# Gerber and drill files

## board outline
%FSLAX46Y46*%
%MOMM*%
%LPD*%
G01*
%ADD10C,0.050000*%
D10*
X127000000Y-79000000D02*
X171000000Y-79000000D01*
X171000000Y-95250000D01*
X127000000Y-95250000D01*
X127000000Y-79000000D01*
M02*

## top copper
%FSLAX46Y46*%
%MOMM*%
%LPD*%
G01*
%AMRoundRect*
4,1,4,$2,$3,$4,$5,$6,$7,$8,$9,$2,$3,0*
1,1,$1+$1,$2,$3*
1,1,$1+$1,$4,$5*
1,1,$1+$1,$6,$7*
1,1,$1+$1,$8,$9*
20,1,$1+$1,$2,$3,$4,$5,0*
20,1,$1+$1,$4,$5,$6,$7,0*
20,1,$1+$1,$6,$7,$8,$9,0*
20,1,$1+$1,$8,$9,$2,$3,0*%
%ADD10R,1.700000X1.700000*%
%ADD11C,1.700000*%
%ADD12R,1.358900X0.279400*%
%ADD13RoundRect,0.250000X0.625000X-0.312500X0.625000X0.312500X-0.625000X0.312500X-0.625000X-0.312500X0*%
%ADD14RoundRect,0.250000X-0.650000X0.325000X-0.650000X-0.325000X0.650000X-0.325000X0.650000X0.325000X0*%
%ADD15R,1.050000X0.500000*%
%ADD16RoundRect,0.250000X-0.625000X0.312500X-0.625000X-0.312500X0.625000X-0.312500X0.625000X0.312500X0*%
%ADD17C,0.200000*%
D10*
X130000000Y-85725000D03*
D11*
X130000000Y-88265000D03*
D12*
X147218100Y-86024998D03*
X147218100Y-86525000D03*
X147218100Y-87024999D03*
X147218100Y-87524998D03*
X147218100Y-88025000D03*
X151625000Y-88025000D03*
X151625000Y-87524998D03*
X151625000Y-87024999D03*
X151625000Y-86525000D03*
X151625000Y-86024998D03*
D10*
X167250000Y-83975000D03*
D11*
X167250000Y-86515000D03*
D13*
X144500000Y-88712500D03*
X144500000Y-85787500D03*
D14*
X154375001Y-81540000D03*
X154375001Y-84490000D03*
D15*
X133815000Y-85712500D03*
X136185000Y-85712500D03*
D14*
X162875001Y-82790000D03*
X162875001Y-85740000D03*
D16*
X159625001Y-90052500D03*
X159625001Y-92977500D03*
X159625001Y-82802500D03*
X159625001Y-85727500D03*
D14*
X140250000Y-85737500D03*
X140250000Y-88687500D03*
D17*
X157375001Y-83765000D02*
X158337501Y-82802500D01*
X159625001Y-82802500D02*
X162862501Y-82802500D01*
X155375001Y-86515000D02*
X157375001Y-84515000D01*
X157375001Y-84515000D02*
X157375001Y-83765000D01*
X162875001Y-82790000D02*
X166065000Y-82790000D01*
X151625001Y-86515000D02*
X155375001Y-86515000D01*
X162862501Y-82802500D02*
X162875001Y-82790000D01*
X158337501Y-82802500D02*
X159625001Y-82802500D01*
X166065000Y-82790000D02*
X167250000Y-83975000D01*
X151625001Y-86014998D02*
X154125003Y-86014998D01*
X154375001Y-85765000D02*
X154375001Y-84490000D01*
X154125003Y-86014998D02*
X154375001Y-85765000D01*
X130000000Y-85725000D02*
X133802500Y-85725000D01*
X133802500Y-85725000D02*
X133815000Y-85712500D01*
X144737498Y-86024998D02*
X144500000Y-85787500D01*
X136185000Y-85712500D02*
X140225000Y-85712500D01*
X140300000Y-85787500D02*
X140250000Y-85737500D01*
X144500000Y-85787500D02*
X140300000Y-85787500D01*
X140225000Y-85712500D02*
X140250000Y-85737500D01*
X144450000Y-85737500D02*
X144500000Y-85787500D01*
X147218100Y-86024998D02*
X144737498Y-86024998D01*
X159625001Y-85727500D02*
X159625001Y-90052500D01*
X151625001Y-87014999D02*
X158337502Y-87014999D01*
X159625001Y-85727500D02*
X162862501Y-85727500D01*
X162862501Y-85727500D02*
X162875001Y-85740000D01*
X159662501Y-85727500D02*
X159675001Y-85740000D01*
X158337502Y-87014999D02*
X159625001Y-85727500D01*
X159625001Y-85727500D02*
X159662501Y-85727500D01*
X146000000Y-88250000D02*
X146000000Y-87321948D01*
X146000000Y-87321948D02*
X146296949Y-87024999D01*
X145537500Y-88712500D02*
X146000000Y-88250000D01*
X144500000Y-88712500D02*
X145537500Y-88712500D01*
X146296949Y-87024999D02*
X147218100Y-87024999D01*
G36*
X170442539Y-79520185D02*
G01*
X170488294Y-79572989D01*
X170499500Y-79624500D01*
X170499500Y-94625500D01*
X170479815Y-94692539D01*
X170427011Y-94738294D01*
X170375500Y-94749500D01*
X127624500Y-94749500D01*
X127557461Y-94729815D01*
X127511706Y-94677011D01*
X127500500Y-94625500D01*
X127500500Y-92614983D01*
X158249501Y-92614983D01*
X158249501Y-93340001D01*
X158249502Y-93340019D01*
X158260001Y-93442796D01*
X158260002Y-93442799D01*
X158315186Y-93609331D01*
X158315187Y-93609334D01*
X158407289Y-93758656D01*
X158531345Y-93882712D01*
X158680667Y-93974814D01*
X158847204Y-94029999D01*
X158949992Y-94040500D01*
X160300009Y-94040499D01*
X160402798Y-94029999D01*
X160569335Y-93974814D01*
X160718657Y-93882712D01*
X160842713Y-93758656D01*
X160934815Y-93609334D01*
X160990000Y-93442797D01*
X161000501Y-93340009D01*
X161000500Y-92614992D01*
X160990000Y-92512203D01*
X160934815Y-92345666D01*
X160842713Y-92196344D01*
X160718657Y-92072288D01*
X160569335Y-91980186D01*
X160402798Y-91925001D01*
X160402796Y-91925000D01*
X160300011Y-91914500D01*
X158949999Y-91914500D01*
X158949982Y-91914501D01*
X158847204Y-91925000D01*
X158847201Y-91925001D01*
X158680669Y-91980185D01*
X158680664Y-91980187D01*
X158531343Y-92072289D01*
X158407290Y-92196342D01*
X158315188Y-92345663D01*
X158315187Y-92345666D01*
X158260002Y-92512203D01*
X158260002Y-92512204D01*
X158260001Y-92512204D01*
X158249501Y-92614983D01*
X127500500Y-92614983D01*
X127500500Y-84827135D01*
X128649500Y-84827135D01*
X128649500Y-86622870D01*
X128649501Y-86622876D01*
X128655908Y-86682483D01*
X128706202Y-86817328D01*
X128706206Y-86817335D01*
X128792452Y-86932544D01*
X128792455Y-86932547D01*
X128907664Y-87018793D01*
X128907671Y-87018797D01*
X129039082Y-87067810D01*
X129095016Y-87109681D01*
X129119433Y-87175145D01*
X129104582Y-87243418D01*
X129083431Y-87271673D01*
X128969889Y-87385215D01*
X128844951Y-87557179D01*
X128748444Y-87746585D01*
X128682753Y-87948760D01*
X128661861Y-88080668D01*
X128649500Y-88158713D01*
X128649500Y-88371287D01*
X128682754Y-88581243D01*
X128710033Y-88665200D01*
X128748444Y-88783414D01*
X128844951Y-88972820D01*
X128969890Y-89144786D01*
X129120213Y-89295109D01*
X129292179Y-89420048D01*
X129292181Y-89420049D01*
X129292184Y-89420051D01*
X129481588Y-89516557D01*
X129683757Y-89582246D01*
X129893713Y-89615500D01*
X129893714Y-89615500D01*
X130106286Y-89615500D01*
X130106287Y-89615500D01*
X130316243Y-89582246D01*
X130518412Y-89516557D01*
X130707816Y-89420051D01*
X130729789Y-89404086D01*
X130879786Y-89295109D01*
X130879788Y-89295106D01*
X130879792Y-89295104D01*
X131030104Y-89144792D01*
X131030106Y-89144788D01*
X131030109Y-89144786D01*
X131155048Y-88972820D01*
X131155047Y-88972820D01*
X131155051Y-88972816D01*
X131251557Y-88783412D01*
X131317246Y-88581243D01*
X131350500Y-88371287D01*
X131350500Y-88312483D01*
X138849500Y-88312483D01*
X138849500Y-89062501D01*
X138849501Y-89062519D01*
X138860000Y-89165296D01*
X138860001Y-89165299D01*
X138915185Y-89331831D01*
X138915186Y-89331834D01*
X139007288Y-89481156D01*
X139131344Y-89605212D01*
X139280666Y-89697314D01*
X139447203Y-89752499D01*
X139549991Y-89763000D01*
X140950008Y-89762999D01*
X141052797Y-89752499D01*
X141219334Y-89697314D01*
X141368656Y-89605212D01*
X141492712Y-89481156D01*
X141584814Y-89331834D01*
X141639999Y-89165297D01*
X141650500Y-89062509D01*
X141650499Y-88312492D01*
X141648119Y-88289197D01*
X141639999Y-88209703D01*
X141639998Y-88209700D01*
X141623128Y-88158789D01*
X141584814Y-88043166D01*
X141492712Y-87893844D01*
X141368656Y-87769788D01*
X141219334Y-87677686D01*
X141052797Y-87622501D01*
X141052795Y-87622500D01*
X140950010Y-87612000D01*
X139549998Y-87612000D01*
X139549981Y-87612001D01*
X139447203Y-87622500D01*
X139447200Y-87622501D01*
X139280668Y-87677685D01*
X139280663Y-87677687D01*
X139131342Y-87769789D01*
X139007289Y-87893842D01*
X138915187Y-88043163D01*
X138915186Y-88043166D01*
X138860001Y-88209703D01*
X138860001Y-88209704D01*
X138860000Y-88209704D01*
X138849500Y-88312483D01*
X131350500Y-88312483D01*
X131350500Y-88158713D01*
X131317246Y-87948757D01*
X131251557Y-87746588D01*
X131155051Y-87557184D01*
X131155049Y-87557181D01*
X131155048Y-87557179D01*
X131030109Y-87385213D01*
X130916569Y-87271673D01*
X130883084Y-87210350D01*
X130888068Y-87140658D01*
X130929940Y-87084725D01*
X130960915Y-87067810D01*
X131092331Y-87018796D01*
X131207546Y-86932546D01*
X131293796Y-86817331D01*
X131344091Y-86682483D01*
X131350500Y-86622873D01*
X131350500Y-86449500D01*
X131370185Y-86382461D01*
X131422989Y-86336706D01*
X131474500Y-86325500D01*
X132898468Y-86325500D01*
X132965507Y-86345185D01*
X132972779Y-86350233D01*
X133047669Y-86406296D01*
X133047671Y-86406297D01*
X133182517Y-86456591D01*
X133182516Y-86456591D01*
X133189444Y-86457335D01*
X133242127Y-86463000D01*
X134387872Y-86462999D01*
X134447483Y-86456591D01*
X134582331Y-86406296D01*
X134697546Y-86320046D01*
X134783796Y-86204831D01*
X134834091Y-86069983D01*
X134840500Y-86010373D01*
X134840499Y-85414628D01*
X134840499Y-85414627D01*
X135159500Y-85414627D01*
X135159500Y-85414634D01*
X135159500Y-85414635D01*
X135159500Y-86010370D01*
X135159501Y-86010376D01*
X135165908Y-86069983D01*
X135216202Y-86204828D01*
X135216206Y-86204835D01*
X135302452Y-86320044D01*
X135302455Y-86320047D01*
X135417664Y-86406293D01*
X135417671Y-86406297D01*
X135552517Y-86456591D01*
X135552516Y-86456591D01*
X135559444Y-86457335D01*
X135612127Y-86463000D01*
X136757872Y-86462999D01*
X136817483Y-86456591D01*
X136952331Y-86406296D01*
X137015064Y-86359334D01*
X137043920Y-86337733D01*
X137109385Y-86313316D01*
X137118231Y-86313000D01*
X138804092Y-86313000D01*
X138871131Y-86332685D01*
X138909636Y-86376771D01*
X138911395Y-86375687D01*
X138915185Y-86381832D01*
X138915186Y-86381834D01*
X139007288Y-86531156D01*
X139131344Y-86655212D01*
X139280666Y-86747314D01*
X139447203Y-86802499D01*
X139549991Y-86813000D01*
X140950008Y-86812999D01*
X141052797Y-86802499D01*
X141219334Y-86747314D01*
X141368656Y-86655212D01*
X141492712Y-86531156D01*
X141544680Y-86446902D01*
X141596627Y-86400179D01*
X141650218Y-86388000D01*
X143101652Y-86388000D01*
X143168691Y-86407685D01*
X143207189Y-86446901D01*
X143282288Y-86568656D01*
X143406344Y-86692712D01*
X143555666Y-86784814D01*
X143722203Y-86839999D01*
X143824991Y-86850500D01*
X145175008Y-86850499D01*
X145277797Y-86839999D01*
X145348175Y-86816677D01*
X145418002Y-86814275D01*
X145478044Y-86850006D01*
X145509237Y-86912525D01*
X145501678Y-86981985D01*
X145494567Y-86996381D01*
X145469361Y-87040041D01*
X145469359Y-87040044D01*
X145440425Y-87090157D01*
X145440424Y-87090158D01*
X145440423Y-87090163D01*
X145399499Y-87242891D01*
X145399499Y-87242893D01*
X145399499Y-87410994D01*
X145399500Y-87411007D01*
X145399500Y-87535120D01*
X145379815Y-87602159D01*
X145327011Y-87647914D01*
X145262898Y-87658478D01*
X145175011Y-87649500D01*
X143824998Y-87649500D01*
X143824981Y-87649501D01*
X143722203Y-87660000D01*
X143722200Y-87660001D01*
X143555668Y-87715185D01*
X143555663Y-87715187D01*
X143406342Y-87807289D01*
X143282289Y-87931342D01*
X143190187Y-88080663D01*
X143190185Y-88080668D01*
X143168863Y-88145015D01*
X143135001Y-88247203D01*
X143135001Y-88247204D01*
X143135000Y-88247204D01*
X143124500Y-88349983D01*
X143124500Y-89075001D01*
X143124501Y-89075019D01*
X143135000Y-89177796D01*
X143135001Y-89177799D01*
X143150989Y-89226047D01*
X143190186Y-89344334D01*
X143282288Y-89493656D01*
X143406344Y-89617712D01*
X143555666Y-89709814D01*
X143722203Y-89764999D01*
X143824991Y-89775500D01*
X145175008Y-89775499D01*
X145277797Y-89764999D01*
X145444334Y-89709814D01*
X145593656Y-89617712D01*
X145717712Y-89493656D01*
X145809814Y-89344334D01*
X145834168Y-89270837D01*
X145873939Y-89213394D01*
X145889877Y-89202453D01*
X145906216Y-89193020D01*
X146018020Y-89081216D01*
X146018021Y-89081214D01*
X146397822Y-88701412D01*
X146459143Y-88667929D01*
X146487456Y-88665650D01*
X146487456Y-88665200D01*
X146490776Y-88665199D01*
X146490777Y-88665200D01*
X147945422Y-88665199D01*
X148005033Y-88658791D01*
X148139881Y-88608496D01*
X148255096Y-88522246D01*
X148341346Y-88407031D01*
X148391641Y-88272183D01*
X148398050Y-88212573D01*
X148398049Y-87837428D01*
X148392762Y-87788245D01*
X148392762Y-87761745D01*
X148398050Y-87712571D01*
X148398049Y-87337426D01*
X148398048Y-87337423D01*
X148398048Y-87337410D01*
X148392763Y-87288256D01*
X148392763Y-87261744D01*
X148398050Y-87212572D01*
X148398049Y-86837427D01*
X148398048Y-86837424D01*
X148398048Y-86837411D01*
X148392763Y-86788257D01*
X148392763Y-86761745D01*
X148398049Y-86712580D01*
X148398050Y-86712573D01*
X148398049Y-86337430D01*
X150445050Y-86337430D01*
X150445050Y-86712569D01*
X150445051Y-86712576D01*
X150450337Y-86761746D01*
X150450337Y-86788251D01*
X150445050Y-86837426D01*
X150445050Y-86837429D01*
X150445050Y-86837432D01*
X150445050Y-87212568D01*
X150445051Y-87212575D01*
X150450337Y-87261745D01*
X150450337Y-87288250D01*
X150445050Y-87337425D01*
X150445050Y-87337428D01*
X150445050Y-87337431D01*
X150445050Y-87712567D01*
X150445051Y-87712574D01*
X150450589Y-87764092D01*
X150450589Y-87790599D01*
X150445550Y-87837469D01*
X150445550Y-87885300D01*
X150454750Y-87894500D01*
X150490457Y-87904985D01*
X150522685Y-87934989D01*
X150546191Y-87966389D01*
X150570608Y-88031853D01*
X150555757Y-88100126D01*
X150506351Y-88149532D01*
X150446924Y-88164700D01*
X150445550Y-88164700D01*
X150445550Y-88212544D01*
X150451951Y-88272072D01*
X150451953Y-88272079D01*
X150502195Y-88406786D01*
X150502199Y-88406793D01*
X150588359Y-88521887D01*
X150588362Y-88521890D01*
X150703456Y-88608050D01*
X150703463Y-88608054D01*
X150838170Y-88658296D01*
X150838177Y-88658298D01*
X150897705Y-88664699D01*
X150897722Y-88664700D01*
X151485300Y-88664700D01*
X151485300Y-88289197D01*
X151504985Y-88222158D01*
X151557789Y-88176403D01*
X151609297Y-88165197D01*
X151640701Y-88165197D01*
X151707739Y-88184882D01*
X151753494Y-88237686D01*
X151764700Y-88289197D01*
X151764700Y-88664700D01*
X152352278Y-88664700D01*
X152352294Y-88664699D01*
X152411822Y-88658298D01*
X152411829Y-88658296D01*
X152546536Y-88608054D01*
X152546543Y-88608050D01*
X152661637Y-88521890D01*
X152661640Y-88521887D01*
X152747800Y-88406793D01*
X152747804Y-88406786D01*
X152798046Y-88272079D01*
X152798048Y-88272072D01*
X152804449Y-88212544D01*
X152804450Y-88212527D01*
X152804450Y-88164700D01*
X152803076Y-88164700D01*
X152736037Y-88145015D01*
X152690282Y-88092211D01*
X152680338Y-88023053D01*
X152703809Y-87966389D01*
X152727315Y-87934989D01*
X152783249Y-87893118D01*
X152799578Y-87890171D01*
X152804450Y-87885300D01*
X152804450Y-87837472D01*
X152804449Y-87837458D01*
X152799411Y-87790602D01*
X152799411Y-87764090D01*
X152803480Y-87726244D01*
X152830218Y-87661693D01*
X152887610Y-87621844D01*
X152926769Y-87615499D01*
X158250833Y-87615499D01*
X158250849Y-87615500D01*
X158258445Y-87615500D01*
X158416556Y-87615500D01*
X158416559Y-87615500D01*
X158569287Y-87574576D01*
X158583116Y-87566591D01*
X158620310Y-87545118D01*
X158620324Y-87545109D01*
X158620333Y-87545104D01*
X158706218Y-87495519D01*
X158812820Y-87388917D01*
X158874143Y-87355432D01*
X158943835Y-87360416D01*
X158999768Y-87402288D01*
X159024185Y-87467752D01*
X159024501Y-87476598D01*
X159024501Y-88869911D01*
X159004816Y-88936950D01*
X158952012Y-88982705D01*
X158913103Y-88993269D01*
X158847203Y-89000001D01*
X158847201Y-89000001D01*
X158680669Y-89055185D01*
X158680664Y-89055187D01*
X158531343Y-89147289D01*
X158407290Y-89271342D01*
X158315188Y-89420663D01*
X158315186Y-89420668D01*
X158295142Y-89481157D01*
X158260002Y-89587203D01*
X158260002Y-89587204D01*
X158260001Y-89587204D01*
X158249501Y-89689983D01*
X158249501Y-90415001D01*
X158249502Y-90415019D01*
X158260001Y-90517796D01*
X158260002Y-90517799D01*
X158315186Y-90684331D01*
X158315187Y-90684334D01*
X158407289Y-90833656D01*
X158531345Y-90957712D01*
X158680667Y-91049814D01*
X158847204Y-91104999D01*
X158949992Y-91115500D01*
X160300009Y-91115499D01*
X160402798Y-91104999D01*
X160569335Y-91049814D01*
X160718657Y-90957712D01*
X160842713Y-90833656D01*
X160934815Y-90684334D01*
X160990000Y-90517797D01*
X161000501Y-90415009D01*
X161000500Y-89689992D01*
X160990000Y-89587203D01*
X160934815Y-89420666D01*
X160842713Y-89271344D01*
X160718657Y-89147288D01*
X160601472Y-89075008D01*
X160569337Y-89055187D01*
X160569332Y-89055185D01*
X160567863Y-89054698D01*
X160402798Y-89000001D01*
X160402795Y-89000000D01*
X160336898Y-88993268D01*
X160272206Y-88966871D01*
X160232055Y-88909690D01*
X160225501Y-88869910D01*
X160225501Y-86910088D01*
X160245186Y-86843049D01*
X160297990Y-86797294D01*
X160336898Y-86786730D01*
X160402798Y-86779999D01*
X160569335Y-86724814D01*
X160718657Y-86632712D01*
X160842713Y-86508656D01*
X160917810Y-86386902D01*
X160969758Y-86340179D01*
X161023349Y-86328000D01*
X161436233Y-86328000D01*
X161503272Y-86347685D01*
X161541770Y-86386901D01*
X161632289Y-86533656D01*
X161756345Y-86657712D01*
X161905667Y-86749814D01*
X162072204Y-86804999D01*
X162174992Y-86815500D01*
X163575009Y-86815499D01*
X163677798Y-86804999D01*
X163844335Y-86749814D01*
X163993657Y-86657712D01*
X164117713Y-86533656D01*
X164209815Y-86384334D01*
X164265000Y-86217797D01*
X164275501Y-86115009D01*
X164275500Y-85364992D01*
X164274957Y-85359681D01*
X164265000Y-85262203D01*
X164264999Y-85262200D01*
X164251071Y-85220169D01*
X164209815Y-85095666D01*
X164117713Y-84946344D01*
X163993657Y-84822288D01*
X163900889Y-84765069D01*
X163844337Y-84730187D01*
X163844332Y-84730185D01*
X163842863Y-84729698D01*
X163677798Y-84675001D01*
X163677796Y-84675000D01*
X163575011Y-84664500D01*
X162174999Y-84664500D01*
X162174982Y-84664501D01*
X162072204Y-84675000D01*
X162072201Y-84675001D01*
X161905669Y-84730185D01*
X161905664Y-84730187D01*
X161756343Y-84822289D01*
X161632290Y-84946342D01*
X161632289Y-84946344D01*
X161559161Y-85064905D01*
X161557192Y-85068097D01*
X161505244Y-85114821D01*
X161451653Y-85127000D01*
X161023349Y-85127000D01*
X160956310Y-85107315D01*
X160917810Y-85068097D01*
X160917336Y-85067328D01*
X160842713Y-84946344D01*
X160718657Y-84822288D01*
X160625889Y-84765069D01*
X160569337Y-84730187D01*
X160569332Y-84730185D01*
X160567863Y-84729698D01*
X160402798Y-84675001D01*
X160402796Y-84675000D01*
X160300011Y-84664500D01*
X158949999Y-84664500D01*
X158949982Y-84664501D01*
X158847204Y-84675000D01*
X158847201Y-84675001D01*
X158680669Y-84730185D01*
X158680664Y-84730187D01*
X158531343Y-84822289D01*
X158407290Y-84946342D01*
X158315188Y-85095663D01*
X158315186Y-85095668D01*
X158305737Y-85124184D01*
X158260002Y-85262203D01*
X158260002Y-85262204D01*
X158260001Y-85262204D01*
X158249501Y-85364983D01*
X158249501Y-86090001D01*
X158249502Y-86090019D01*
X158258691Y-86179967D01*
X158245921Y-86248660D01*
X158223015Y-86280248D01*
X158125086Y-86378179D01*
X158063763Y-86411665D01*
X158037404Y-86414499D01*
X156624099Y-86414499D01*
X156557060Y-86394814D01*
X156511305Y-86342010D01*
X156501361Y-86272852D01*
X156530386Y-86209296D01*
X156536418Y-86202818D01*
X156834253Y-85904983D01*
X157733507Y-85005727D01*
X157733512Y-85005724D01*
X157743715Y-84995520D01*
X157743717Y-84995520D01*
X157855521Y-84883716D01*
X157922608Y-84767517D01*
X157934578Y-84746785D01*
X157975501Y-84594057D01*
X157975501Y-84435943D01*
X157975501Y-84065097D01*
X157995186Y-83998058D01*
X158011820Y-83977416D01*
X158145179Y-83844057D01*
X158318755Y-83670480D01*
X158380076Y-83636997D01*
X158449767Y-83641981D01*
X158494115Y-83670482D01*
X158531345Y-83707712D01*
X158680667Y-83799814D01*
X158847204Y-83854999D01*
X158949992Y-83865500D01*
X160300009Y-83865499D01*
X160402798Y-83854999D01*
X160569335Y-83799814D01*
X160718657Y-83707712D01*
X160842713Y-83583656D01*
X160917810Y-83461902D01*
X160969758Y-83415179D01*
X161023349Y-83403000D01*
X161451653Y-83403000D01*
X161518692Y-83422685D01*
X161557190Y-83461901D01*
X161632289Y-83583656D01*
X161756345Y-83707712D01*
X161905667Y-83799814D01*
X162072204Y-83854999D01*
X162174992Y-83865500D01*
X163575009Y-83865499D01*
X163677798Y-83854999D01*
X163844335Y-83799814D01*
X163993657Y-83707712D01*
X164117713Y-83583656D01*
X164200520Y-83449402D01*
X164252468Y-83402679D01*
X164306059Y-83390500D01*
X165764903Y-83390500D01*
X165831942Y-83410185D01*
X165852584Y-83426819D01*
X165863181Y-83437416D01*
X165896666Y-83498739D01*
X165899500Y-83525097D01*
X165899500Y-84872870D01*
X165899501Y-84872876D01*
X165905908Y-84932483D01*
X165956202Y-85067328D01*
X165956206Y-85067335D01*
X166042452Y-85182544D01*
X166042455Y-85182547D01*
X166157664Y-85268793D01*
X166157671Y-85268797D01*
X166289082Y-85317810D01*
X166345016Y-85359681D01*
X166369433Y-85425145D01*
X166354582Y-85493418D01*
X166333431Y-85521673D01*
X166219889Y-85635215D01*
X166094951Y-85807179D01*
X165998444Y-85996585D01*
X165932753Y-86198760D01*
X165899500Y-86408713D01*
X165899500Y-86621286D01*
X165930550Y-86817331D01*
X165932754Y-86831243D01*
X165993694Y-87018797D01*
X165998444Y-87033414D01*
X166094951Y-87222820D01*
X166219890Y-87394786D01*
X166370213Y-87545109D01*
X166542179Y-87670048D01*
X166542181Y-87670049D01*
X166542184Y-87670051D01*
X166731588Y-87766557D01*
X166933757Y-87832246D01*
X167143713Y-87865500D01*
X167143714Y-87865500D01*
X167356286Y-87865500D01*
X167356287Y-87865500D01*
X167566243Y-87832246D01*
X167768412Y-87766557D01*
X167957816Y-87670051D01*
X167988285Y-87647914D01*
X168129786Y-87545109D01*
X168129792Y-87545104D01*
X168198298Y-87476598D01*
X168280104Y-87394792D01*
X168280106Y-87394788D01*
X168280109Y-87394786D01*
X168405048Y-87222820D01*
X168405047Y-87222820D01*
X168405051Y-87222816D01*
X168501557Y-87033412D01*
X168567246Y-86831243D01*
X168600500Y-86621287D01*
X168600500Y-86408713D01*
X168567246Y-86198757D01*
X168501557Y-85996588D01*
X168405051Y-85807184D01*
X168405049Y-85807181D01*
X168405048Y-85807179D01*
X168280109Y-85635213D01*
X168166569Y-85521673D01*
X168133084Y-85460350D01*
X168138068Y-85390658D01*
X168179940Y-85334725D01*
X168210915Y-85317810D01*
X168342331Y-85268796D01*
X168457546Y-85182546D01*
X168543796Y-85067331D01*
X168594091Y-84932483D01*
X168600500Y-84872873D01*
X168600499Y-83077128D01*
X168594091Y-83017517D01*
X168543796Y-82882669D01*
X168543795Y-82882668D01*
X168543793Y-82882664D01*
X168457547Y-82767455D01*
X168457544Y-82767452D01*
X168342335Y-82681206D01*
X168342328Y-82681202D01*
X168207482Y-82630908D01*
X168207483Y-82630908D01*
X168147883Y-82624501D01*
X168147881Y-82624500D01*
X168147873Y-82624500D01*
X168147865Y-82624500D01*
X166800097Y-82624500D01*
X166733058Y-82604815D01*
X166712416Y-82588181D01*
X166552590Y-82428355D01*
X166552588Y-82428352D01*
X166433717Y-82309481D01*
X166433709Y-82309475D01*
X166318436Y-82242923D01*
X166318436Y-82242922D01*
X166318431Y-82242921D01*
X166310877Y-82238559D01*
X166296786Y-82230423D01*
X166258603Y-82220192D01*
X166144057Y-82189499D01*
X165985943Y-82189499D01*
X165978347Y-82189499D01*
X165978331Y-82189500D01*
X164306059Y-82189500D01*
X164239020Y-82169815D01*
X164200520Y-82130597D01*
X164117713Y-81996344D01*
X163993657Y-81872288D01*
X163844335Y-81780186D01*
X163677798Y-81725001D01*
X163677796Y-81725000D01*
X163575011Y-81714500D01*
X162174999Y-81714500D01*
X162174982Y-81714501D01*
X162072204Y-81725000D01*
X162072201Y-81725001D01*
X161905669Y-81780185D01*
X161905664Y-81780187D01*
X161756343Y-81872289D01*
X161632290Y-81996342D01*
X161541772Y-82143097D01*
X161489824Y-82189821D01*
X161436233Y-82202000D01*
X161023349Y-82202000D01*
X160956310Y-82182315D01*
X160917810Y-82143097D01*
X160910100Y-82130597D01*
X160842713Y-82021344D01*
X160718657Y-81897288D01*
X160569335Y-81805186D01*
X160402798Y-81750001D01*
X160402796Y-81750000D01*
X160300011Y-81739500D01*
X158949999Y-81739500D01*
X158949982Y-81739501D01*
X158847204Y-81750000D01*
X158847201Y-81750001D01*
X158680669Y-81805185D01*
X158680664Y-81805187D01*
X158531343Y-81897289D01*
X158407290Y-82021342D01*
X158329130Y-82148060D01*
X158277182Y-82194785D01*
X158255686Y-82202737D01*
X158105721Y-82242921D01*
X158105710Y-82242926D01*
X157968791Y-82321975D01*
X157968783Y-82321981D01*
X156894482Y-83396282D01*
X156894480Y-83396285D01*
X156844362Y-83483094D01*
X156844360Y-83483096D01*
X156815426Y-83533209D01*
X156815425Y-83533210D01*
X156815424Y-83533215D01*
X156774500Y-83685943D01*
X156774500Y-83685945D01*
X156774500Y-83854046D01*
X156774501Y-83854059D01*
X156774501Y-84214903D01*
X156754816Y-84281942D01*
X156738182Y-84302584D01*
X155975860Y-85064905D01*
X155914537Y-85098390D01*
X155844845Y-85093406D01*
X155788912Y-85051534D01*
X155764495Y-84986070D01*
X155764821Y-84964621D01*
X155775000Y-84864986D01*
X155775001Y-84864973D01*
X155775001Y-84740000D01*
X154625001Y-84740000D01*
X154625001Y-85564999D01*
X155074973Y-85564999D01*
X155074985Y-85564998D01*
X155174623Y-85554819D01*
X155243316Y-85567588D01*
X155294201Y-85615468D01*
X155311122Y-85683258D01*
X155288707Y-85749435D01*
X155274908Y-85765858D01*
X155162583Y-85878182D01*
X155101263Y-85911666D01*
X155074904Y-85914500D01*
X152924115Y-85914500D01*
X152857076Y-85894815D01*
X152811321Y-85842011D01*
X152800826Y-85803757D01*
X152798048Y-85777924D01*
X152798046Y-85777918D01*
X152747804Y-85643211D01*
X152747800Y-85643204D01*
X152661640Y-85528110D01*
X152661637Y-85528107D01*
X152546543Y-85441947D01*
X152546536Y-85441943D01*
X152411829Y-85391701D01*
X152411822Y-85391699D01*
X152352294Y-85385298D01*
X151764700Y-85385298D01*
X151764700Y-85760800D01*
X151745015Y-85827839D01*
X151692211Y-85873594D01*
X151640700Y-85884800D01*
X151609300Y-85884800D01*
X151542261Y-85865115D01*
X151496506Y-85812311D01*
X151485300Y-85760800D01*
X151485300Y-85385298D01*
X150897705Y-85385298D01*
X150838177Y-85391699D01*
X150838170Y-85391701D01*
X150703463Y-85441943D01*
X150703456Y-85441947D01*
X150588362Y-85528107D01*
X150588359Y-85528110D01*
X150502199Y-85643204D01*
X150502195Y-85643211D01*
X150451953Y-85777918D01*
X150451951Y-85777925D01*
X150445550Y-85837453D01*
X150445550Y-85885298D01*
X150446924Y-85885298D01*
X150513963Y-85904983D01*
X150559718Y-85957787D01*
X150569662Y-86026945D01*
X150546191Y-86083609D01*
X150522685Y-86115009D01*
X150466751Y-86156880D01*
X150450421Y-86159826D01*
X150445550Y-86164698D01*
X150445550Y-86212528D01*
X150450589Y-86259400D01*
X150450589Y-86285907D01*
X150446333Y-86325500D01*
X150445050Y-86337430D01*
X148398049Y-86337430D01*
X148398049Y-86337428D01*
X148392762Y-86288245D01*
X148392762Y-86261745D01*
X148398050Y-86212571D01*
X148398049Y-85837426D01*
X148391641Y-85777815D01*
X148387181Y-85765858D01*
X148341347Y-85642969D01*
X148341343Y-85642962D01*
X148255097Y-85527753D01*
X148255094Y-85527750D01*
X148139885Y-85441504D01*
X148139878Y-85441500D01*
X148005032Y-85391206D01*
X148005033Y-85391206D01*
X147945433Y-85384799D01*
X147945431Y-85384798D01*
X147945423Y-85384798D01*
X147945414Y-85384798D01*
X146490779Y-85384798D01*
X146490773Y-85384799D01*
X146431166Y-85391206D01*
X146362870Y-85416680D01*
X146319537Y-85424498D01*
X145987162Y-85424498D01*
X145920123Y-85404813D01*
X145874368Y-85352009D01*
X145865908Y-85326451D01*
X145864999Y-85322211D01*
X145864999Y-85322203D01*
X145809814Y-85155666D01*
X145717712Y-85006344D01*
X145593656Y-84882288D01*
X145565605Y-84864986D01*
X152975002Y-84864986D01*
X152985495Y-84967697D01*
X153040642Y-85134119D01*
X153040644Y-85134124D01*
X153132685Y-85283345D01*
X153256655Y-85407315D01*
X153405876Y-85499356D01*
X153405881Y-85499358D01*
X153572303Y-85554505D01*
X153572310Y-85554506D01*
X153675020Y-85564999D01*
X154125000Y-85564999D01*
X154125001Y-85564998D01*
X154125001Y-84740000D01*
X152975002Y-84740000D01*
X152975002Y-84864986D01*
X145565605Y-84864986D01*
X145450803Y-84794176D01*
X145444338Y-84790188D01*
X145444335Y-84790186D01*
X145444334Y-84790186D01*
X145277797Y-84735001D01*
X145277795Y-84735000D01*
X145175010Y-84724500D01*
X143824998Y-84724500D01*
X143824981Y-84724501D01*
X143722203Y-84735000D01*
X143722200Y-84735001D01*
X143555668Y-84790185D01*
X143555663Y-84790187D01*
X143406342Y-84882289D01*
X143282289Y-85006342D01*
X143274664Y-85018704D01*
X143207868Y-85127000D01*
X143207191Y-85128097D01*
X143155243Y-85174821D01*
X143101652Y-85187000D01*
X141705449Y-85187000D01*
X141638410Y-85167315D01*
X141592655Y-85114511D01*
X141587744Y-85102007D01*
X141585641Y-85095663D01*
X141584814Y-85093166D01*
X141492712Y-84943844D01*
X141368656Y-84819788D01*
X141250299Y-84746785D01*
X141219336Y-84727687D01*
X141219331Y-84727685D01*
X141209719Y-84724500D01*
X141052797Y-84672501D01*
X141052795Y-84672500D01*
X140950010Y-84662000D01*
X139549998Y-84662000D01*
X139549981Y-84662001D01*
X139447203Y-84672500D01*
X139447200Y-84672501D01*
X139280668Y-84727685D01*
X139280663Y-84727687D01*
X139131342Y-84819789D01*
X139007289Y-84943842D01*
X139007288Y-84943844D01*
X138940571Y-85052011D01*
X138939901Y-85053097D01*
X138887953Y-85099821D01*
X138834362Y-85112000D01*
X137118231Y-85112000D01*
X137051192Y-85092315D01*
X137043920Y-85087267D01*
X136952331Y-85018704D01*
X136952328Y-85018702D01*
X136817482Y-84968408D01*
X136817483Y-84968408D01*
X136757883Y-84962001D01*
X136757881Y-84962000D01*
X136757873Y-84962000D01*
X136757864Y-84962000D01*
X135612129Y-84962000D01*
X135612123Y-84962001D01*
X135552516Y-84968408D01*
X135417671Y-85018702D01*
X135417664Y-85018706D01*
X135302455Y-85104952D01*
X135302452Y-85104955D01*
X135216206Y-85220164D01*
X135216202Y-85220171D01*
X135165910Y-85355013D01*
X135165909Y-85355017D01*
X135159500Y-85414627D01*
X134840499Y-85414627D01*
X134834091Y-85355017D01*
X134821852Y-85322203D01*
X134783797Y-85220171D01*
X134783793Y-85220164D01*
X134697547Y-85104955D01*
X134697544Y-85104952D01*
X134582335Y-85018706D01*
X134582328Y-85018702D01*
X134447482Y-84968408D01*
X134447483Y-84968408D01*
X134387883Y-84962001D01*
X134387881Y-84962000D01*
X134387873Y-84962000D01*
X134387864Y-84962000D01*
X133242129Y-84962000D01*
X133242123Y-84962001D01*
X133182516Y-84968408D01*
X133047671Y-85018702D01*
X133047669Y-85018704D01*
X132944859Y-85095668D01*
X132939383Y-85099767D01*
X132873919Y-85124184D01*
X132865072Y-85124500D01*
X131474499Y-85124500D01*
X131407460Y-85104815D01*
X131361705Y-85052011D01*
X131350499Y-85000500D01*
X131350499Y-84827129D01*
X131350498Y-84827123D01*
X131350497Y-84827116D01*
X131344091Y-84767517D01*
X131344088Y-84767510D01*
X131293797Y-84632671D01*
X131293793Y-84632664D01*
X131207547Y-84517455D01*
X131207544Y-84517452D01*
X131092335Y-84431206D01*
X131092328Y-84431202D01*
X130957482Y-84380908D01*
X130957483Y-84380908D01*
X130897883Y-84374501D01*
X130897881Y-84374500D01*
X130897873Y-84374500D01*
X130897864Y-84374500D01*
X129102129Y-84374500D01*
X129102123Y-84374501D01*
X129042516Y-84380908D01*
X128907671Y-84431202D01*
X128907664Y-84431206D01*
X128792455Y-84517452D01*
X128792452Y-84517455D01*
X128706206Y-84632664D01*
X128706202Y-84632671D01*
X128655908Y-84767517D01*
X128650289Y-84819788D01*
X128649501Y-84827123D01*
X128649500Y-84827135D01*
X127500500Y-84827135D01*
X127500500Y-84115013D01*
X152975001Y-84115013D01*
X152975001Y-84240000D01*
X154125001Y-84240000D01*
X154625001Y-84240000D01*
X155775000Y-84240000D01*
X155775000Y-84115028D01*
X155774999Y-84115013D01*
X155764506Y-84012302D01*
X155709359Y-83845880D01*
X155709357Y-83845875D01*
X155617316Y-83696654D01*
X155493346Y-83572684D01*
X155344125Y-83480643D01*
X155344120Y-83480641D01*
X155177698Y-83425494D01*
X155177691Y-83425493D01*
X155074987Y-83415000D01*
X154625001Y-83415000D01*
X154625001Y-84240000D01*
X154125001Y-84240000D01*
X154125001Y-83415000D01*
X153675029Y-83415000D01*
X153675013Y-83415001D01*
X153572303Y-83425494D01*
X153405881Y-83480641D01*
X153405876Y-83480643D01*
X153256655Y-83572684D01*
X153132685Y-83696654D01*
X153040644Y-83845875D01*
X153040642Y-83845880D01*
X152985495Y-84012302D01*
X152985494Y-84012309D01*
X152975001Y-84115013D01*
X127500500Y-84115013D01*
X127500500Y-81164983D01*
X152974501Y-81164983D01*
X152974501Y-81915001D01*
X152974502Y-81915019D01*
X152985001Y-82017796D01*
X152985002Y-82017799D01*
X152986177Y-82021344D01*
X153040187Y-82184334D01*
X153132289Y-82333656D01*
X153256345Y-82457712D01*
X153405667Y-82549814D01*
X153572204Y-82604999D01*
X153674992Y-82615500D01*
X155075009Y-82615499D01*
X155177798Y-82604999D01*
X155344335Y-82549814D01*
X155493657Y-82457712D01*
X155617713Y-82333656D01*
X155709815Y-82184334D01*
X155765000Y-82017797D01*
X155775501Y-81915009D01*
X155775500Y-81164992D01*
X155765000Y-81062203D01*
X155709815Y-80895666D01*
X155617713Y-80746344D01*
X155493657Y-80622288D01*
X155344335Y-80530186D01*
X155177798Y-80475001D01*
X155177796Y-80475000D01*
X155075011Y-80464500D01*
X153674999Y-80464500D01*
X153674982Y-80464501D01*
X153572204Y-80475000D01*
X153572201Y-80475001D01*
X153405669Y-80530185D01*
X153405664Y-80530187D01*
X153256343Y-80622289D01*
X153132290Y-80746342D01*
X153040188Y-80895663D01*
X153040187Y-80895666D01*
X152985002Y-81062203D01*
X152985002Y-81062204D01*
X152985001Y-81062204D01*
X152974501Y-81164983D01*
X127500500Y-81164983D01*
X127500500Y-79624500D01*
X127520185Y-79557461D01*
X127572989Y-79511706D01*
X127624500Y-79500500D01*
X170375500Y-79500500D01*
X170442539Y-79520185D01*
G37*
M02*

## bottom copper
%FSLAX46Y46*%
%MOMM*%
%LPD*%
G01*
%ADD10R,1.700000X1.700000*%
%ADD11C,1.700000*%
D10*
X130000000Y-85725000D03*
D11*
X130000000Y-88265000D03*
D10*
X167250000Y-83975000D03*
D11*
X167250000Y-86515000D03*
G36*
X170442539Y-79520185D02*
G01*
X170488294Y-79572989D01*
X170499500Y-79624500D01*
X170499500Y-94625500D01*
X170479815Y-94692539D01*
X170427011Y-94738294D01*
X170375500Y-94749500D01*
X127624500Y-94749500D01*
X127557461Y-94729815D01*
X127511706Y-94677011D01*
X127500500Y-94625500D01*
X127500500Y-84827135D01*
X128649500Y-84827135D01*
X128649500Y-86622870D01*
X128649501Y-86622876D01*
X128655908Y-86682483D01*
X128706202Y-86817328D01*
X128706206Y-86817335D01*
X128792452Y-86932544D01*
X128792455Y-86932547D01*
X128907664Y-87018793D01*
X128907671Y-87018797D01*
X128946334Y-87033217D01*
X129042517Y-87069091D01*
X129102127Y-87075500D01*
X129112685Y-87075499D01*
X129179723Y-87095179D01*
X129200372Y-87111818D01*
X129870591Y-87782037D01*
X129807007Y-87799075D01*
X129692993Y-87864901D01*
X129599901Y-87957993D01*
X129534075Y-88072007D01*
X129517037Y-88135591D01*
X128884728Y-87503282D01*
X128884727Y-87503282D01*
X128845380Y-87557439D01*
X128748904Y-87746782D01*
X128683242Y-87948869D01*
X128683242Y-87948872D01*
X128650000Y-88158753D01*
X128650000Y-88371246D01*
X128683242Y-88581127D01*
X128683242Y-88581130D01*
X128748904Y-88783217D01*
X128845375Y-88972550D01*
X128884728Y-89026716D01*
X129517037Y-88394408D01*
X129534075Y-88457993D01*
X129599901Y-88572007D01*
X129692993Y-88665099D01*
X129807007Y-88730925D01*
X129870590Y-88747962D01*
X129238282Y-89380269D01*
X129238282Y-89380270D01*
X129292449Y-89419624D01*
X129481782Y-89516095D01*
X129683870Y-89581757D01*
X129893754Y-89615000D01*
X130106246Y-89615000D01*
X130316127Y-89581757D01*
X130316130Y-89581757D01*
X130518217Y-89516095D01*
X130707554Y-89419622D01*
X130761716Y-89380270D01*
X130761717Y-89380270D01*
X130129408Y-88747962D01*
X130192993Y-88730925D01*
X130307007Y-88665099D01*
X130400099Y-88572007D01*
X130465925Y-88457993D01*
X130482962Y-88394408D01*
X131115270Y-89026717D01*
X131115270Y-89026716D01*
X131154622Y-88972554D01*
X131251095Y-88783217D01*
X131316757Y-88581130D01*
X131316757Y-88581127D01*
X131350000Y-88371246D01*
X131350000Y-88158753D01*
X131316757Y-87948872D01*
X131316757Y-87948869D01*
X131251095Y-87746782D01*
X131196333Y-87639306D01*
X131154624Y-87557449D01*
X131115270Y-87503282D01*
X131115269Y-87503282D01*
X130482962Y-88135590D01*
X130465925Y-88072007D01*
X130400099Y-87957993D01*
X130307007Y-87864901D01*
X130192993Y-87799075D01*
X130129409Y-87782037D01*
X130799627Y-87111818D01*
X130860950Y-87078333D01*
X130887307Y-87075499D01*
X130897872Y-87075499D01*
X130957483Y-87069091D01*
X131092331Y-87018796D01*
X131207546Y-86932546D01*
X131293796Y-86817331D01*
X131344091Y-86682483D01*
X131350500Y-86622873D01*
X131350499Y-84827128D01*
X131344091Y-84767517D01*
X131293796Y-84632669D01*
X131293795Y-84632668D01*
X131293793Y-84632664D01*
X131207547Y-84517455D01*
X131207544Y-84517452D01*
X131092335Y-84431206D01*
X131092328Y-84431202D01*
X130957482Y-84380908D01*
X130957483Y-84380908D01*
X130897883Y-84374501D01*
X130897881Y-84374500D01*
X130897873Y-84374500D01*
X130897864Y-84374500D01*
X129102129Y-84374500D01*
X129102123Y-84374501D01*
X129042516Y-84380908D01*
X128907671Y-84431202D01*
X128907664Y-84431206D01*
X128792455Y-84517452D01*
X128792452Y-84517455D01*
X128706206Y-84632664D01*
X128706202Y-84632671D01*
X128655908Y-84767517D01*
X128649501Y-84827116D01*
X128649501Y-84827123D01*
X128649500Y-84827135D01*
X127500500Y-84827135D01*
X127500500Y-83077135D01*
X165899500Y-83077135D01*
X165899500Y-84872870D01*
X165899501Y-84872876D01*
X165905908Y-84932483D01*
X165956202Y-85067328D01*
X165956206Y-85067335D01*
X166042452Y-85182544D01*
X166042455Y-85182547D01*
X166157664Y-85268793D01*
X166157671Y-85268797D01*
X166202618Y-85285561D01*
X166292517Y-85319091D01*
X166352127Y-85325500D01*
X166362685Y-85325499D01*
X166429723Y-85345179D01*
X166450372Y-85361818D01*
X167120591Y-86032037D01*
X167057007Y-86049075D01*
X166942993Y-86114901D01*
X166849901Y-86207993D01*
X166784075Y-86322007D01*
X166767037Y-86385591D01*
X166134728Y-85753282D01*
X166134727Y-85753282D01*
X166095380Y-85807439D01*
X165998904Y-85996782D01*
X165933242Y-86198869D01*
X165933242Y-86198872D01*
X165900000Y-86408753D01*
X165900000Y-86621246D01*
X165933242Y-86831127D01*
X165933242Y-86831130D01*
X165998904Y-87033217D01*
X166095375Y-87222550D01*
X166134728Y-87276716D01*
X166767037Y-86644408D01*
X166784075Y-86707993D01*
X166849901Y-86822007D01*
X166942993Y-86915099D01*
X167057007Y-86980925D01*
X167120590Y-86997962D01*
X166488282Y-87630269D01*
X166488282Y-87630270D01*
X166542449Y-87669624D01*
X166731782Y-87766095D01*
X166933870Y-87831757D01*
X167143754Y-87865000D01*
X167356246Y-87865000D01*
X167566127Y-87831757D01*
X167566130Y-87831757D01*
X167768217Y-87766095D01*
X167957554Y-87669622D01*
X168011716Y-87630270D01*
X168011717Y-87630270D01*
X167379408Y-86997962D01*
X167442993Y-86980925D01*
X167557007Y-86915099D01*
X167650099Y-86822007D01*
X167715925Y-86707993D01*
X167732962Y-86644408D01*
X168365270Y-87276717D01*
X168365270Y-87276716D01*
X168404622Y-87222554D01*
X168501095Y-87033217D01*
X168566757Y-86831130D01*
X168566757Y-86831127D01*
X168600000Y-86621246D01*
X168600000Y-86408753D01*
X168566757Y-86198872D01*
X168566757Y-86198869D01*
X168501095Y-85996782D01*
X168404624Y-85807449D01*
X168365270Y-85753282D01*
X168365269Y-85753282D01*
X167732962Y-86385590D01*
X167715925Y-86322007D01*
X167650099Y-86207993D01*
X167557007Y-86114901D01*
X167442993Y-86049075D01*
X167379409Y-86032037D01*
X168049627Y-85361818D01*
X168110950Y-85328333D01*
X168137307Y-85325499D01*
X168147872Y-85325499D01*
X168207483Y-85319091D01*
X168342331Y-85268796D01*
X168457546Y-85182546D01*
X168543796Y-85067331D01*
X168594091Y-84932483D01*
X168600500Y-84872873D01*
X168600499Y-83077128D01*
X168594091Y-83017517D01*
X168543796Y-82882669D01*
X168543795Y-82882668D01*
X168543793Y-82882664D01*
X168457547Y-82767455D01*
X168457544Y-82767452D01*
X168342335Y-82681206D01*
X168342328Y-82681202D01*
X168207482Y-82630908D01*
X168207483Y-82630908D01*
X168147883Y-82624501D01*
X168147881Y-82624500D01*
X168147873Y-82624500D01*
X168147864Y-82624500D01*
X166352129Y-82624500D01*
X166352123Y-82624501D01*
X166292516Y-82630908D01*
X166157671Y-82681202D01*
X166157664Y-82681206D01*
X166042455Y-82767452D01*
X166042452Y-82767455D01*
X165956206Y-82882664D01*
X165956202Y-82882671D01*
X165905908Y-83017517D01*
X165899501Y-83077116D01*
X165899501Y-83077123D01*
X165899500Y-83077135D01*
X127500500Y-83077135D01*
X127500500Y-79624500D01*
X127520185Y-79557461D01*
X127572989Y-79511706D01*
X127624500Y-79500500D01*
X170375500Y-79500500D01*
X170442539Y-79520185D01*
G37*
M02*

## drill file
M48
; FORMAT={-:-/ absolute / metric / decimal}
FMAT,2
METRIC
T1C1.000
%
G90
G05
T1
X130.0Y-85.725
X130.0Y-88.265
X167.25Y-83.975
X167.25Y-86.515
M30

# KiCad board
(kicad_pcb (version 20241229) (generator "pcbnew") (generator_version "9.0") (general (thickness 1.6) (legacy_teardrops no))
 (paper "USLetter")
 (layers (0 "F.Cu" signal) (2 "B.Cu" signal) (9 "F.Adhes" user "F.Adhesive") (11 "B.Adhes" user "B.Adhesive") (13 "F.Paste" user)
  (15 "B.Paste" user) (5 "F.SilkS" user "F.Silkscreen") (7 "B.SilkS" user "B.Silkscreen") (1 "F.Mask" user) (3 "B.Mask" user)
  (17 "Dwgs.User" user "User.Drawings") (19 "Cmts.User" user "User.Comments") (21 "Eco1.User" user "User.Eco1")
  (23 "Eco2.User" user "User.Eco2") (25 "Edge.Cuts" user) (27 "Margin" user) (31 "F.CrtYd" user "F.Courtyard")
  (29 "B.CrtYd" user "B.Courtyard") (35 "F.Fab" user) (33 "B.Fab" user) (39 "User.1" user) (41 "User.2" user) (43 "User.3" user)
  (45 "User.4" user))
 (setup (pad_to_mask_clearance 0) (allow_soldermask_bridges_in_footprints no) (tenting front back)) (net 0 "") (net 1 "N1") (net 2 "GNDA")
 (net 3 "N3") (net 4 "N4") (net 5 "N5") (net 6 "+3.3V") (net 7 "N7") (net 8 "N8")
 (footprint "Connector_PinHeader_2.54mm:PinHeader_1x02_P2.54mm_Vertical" (layer "F.Cu") (at 130 85.725)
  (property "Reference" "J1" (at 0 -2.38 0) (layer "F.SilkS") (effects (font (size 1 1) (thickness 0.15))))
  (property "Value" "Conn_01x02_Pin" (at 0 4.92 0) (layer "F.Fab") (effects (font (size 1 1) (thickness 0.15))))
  (pad "1" thru_hole rect (at 0 0) (size 1.7 1.7) (drill 1) (layers "*.Cu" "*.Mask") (remove_unused_layers no) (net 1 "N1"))
  (pad "2" thru_hole circle (at 0 2.54) (size 1.7 1.7) (drill 1) (layers "*.Cu" "*.Mask") (remove_unused_layers no) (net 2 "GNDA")))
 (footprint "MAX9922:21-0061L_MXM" (layer "F.Cu") (at 149.42155 87.024999)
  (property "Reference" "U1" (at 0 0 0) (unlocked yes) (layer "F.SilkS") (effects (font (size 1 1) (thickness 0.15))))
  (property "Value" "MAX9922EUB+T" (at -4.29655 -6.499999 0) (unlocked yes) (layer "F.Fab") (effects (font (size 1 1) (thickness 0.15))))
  (pad "1" smd rect (at -2.20345 -1.000001) (size 1.3589 0.2794) (layers "F.Cu" "F.Mask" "F.Paste") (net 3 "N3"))
  (pad "2" smd rect (at -2.20345 -0.499999) (size 1.3589 0.2794) (layers "F.Cu" "F.Mask" "F.Paste") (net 3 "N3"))
  (pad "3" smd rect (at -2.20345 0) (size 1.3589 0.2794) (layers "F.Cu" "F.Mask" "F.Paste") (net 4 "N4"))
  (pad "4" smd rect (at -2.20345 0.499999) (size 1.3589 0.2794) (layers "F.Cu" "F.Mask" "F.Paste") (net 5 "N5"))
  (pad "5" smd rect (at -2.20345 1.000001) (size 1.3589 0.2794) (layers "F.Cu" "F.Mask" "F.Paste") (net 2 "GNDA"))
  (pad "6" smd rect (at 2.20345 1.000001) (size 1.3589 0.2794) (layers "F.Cu" "F.Mask" "F.Paste") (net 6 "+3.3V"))
  (pad "7" smd rect (at 2.20345 0.499999) (size 1.3589 0.2794) (layers "F.Cu" "F.Mask" "F.Paste") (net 2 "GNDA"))
  (pad "8" smd rect (at 2.20345 0) (size 1.3589 0.2794) (layers "F.Cu" "F.Mask" "F.Paste") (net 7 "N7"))
  (pad "9" smd rect (at 2.20345 -0.499999) (size 1.3589 0.2794) (layers "F.Cu" "F.Mask" "F.Paste") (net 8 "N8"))
  (pad "10" smd rect (at 2.20345 -1.000001) (size 1.3589 0.2794) (layers "F.Cu" "F.Mask" "F.Paste") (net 6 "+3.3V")))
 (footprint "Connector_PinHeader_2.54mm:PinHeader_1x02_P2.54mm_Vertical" (layer "F.Cu") (at 167.25 83.975)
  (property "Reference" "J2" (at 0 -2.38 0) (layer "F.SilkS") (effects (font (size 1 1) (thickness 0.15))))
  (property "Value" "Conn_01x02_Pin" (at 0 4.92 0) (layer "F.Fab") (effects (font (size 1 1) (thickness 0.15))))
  (pad "1" thru_hole rect (at 0 0) (size 1.7 1.7) (drill 1) (layers "*.Cu" "*.Mask") (remove_unused_layers no) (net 8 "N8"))
  (pad "2" thru_hole circle (at 0 2.54) (size 1.7 1.7) (drill 1) (layers "*.Cu" "*.Mask") (remove_unused_layers no) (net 2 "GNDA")))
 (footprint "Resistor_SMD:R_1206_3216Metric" (layer "F.Cu") (at 144.5 87.25 90)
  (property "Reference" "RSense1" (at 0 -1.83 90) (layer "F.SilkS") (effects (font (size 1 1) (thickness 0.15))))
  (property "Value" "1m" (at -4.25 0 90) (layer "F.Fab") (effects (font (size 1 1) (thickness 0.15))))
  (pad "1" smd roundrect (at -1.4625 0 90) (size 1.125 1.75) (layers "F.Cu" "F.Mask" "F.Paste") (roundrect_rratio 0.222222) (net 4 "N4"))
  (pad "2" smd roundrect (at 1.4625 0 90) (size 1.125 1.75) (layers "F.Cu" "F.Mask" "F.Paste") (roundrect_rratio 0.222222) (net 3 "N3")))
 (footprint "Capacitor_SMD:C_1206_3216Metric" (layer "F.Cu") (at 154.375001 83.015 -90)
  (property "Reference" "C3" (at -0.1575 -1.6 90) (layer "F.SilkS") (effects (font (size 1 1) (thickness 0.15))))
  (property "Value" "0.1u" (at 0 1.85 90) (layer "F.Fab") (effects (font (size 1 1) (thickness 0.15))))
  (pad "1" smd roundrect (at -1.475 0 270) (size 1.15 1.8) (layers "F.Cu" "F.Mask" "F.Paste") (roundrect_rratio 0.217391) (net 2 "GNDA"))
  (pad "2" smd roundrect (at 1.475 0 270) (size 1.15 1.8) (layers "F.Cu" "F.Mask" "F.Paste") (roundrect_rratio 0.217391) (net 6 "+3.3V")))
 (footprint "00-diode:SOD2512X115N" (layer "F.Cu") (at 135 85.7125 180)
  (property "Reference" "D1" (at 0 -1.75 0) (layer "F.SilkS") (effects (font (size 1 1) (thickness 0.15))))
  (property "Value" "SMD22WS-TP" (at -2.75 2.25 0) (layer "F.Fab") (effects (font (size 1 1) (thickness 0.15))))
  (pad "A" smd rect (at 1.185 0 180) (size 1.05 0.5) (layers "F.Cu" "F.Mask" "F.Paste") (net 1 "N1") (solder_mask_margin 0.102))
  (pad "C" smd rect (at -1.185 0 180) (size 1.05 0.5) (layers "F.Cu" "F.Mask" "F.Paste") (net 3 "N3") (solder_mask_margin 0.102)))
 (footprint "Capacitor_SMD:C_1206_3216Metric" (layer "F.Cu") (at 162.875001 84.265 -90)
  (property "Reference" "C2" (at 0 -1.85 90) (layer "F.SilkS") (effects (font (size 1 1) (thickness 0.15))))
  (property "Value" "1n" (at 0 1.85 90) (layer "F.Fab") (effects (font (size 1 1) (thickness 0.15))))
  (pad "1" smd roundrect (at -1.475 0 270) (size 1.15 1.8) (layers "F.Cu" "F.Mask" "F.Paste") (roundrect_rratio 0.217391) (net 8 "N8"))
  (pad "2" smd roundrect (at 1.475 0 270) (size 1.15 1.8) (layers "F.Cu" "F.Mask" "F.Paste") (roundrect_rratio 0.217391) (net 7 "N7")))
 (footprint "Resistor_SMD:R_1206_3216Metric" (layer "F.Cu") (at 159.625001 91.515 -90)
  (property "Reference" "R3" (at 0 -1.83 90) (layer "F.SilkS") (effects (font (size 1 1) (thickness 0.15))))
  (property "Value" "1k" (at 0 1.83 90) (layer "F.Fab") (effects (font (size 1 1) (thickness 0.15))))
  (pad "1" smd roundrect (at -1.4625 0 270) (size 1.125 1.75) (layers "F.Cu" "F.Mask" "F.Paste") (roundrect_rratio 0.222222) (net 7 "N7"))
  (pad "2" smd roundrect (at 1.4625 0 270) (size 1.125 1.75) (layers "F.Cu" "F.Mask" "F.Paste") (roundrect_rratio 0.222222) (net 2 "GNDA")))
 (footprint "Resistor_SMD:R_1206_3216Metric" (layer "F.Cu") (at 159.625001 84.265 -90)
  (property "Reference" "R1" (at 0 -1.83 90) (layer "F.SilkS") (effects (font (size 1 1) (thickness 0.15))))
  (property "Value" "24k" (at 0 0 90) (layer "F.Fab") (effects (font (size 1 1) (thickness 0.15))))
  (pad "1" smd roundrect (at -1.4625 0 270) (size 1.125 1.75) (layers "F.Cu" "F.Mask" "F.Paste") (roundrect_rratio 0.222222) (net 8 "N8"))
  (pad "2" smd roundrect (at 1.4625 0 270) (size 1.125 1.75) (layers "F.Cu" "F.Mask" "F.Paste") (roundrect_rratio 0.222222) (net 7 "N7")))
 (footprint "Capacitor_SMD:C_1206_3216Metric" (layer "F.Cu") (at 140.25 87.2125 -90)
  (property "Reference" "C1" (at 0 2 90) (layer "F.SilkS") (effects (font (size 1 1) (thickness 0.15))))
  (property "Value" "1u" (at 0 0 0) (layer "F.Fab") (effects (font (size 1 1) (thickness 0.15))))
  (pad "1" smd roundrect (at -1.475 0 270) (size 1.15 1.8) (layers "F.Cu" "F.Mask" "F.Paste") (roundrect_rratio 0.217391) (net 3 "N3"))
  (pad "2" smd roundrect (at 1.475 0 270) (size 1.15 1.8) (layers "F.Cu" "F.Mask" "F.Paste") (roundrect_rratio 0.217391) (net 2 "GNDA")))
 (gr_rect (start 127 79) (end 171 95.25) (stroke (width 0.05) (type default)) (fill no) (layer "Edge.Cuts"))
 (segment (start 157.375001 83.765) (end 158.337501 82.8025) (width 0.2) (layer "F.Cu") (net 8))
 (segment (start 159.625001 82.8025) (end 162.862501 82.8025) (width 0.2) (layer "F.Cu") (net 8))
 (segment (start 155.375001 86.515) (end 157.375001 84.515) (width 0.2) (layer "F.Cu") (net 8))
 (segment (start 157.375001 84.515) (end 157.375001 83.765) (width 0.2) (layer "F.Cu") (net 8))
 (segment (start 162.875001 82.79) (end 166.065 82.79) (width 0.2) (layer "F.Cu") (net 8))
 (segment (start 151.625001 86.515) (end 155.375001 86.515) (width 0.2) (layer "F.Cu") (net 8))
 (segment (start 162.862501 82.8025) (end 162.875001 82.79) (width 0.2) (layer "F.Cu") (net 8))
 (segment (start 158.337501 82.8025) (end 159.625001 82.8025) (width 0.2) (layer "F.Cu") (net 8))
 (segment (start 166.065 82.79) (end 167.25 83.975) (width 0.2) (layer "F.Cu") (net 8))
 (segment (start 151.625001 86.014998) (end 154.125003 86.014998) (width 0.2) (layer "F.Cu") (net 6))
 (segment (start 154.375001 85.765) (end 154.375001 84.49) (width 0.2) (layer "F.Cu") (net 6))
 (segment (start 154.125003 86.014998) (end 154.375001 85.765) (width 0.2) (layer "F.Cu") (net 6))
 (segment (start 130 85.725) (end 133.8025 85.725) (width 0.2) (layer "F.Cu") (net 1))
 (segment (start 133.8025 85.725) (end 133.815 85.7125) (width 0.2) (layer "F.Cu") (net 1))
 (segment (start 144.737498 86.024998) (end 144.5 85.7875) (width 0.2) (layer "F.Cu") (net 3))
 (segment (start 136.185 85.7125) (end 140.225 85.7125) (width 0.2) (layer "F.Cu") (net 3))
 (segment (start 140.3 85.7875) (end 140.25 85.7375) (width 0.2) (layer "F.Cu") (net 3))
 (segment (start 144.5 85.7875) (end 140.3 85.7875) (width 0.2) (layer "F.Cu") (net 3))
 (segment (start 140.225 85.7125) (end 140.25 85.7375) (width 0.2) (layer "F.Cu") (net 3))
 (segment (start 144.45 85.7375) (end 144.5 85.7875) (width 0.2) (layer "F.Cu") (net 3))
 (segment (start 147.2181 86.024998) (end 144.737498 86.024998) (width 0.2) (layer "F.Cu") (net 3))
 (segment (start 159.625001 85.7275) (end 159.625001 90.0525) (width 0.2) (layer "F.Cu") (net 7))
 (segment (start 151.625001 87.014999) (end 158.337502 87.014999) (width 0.2) (layer "F.Cu") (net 7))
 (segment (start 159.625001 85.7275) (end 162.862501 85.7275) (width 0.2) (layer "F.Cu") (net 7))
 (segment (start 162.862501 85.7275) (end 162.875001 85.74) (width 0.2) (layer "F.Cu") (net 7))
 (segment (start 159.662501 85.7275) (end 159.675001 85.74) (width 0.2) (layer "F.Cu") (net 7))
 (segment (start 158.337502 87.014999) (end 159.625001 85.7275) (width 0.2) (layer "F.Cu") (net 7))
 (segment (start 159.625001 85.7275) (end 159.662501 85.7275) (width 0.2) (layer "F.Cu") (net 7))
 (segment (start 146 88.25) (end 146 87.321948) (width 0.2) (layer "F.Cu") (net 4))
 (segment (start 146 87.321948) (end 146.296949 87.024999) (width 0.2) (layer "F.Cu") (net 4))
 (segment (start 145.5375 88.7125) (end 146 88.25) (width 0.2) (layer "F.Cu") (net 4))
 (segment (start 144.5 88.7125) (end 145.5375 88.7125) (width 0.2) (layer "F.Cu") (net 4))
 (segment (start 146.296949 87.024999) (end 147.2181 87.024999) (width 0.2) (layer "F.Cu") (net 4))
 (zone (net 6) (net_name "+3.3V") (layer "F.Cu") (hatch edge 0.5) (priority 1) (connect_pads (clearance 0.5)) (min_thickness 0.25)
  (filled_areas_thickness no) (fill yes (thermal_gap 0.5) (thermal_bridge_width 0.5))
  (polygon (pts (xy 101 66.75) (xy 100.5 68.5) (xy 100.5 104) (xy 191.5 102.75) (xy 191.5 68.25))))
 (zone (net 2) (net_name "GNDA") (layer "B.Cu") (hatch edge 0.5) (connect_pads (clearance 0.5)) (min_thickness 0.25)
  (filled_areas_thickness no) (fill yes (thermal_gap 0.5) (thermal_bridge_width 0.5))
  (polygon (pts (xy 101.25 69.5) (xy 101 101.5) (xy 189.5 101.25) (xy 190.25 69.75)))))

